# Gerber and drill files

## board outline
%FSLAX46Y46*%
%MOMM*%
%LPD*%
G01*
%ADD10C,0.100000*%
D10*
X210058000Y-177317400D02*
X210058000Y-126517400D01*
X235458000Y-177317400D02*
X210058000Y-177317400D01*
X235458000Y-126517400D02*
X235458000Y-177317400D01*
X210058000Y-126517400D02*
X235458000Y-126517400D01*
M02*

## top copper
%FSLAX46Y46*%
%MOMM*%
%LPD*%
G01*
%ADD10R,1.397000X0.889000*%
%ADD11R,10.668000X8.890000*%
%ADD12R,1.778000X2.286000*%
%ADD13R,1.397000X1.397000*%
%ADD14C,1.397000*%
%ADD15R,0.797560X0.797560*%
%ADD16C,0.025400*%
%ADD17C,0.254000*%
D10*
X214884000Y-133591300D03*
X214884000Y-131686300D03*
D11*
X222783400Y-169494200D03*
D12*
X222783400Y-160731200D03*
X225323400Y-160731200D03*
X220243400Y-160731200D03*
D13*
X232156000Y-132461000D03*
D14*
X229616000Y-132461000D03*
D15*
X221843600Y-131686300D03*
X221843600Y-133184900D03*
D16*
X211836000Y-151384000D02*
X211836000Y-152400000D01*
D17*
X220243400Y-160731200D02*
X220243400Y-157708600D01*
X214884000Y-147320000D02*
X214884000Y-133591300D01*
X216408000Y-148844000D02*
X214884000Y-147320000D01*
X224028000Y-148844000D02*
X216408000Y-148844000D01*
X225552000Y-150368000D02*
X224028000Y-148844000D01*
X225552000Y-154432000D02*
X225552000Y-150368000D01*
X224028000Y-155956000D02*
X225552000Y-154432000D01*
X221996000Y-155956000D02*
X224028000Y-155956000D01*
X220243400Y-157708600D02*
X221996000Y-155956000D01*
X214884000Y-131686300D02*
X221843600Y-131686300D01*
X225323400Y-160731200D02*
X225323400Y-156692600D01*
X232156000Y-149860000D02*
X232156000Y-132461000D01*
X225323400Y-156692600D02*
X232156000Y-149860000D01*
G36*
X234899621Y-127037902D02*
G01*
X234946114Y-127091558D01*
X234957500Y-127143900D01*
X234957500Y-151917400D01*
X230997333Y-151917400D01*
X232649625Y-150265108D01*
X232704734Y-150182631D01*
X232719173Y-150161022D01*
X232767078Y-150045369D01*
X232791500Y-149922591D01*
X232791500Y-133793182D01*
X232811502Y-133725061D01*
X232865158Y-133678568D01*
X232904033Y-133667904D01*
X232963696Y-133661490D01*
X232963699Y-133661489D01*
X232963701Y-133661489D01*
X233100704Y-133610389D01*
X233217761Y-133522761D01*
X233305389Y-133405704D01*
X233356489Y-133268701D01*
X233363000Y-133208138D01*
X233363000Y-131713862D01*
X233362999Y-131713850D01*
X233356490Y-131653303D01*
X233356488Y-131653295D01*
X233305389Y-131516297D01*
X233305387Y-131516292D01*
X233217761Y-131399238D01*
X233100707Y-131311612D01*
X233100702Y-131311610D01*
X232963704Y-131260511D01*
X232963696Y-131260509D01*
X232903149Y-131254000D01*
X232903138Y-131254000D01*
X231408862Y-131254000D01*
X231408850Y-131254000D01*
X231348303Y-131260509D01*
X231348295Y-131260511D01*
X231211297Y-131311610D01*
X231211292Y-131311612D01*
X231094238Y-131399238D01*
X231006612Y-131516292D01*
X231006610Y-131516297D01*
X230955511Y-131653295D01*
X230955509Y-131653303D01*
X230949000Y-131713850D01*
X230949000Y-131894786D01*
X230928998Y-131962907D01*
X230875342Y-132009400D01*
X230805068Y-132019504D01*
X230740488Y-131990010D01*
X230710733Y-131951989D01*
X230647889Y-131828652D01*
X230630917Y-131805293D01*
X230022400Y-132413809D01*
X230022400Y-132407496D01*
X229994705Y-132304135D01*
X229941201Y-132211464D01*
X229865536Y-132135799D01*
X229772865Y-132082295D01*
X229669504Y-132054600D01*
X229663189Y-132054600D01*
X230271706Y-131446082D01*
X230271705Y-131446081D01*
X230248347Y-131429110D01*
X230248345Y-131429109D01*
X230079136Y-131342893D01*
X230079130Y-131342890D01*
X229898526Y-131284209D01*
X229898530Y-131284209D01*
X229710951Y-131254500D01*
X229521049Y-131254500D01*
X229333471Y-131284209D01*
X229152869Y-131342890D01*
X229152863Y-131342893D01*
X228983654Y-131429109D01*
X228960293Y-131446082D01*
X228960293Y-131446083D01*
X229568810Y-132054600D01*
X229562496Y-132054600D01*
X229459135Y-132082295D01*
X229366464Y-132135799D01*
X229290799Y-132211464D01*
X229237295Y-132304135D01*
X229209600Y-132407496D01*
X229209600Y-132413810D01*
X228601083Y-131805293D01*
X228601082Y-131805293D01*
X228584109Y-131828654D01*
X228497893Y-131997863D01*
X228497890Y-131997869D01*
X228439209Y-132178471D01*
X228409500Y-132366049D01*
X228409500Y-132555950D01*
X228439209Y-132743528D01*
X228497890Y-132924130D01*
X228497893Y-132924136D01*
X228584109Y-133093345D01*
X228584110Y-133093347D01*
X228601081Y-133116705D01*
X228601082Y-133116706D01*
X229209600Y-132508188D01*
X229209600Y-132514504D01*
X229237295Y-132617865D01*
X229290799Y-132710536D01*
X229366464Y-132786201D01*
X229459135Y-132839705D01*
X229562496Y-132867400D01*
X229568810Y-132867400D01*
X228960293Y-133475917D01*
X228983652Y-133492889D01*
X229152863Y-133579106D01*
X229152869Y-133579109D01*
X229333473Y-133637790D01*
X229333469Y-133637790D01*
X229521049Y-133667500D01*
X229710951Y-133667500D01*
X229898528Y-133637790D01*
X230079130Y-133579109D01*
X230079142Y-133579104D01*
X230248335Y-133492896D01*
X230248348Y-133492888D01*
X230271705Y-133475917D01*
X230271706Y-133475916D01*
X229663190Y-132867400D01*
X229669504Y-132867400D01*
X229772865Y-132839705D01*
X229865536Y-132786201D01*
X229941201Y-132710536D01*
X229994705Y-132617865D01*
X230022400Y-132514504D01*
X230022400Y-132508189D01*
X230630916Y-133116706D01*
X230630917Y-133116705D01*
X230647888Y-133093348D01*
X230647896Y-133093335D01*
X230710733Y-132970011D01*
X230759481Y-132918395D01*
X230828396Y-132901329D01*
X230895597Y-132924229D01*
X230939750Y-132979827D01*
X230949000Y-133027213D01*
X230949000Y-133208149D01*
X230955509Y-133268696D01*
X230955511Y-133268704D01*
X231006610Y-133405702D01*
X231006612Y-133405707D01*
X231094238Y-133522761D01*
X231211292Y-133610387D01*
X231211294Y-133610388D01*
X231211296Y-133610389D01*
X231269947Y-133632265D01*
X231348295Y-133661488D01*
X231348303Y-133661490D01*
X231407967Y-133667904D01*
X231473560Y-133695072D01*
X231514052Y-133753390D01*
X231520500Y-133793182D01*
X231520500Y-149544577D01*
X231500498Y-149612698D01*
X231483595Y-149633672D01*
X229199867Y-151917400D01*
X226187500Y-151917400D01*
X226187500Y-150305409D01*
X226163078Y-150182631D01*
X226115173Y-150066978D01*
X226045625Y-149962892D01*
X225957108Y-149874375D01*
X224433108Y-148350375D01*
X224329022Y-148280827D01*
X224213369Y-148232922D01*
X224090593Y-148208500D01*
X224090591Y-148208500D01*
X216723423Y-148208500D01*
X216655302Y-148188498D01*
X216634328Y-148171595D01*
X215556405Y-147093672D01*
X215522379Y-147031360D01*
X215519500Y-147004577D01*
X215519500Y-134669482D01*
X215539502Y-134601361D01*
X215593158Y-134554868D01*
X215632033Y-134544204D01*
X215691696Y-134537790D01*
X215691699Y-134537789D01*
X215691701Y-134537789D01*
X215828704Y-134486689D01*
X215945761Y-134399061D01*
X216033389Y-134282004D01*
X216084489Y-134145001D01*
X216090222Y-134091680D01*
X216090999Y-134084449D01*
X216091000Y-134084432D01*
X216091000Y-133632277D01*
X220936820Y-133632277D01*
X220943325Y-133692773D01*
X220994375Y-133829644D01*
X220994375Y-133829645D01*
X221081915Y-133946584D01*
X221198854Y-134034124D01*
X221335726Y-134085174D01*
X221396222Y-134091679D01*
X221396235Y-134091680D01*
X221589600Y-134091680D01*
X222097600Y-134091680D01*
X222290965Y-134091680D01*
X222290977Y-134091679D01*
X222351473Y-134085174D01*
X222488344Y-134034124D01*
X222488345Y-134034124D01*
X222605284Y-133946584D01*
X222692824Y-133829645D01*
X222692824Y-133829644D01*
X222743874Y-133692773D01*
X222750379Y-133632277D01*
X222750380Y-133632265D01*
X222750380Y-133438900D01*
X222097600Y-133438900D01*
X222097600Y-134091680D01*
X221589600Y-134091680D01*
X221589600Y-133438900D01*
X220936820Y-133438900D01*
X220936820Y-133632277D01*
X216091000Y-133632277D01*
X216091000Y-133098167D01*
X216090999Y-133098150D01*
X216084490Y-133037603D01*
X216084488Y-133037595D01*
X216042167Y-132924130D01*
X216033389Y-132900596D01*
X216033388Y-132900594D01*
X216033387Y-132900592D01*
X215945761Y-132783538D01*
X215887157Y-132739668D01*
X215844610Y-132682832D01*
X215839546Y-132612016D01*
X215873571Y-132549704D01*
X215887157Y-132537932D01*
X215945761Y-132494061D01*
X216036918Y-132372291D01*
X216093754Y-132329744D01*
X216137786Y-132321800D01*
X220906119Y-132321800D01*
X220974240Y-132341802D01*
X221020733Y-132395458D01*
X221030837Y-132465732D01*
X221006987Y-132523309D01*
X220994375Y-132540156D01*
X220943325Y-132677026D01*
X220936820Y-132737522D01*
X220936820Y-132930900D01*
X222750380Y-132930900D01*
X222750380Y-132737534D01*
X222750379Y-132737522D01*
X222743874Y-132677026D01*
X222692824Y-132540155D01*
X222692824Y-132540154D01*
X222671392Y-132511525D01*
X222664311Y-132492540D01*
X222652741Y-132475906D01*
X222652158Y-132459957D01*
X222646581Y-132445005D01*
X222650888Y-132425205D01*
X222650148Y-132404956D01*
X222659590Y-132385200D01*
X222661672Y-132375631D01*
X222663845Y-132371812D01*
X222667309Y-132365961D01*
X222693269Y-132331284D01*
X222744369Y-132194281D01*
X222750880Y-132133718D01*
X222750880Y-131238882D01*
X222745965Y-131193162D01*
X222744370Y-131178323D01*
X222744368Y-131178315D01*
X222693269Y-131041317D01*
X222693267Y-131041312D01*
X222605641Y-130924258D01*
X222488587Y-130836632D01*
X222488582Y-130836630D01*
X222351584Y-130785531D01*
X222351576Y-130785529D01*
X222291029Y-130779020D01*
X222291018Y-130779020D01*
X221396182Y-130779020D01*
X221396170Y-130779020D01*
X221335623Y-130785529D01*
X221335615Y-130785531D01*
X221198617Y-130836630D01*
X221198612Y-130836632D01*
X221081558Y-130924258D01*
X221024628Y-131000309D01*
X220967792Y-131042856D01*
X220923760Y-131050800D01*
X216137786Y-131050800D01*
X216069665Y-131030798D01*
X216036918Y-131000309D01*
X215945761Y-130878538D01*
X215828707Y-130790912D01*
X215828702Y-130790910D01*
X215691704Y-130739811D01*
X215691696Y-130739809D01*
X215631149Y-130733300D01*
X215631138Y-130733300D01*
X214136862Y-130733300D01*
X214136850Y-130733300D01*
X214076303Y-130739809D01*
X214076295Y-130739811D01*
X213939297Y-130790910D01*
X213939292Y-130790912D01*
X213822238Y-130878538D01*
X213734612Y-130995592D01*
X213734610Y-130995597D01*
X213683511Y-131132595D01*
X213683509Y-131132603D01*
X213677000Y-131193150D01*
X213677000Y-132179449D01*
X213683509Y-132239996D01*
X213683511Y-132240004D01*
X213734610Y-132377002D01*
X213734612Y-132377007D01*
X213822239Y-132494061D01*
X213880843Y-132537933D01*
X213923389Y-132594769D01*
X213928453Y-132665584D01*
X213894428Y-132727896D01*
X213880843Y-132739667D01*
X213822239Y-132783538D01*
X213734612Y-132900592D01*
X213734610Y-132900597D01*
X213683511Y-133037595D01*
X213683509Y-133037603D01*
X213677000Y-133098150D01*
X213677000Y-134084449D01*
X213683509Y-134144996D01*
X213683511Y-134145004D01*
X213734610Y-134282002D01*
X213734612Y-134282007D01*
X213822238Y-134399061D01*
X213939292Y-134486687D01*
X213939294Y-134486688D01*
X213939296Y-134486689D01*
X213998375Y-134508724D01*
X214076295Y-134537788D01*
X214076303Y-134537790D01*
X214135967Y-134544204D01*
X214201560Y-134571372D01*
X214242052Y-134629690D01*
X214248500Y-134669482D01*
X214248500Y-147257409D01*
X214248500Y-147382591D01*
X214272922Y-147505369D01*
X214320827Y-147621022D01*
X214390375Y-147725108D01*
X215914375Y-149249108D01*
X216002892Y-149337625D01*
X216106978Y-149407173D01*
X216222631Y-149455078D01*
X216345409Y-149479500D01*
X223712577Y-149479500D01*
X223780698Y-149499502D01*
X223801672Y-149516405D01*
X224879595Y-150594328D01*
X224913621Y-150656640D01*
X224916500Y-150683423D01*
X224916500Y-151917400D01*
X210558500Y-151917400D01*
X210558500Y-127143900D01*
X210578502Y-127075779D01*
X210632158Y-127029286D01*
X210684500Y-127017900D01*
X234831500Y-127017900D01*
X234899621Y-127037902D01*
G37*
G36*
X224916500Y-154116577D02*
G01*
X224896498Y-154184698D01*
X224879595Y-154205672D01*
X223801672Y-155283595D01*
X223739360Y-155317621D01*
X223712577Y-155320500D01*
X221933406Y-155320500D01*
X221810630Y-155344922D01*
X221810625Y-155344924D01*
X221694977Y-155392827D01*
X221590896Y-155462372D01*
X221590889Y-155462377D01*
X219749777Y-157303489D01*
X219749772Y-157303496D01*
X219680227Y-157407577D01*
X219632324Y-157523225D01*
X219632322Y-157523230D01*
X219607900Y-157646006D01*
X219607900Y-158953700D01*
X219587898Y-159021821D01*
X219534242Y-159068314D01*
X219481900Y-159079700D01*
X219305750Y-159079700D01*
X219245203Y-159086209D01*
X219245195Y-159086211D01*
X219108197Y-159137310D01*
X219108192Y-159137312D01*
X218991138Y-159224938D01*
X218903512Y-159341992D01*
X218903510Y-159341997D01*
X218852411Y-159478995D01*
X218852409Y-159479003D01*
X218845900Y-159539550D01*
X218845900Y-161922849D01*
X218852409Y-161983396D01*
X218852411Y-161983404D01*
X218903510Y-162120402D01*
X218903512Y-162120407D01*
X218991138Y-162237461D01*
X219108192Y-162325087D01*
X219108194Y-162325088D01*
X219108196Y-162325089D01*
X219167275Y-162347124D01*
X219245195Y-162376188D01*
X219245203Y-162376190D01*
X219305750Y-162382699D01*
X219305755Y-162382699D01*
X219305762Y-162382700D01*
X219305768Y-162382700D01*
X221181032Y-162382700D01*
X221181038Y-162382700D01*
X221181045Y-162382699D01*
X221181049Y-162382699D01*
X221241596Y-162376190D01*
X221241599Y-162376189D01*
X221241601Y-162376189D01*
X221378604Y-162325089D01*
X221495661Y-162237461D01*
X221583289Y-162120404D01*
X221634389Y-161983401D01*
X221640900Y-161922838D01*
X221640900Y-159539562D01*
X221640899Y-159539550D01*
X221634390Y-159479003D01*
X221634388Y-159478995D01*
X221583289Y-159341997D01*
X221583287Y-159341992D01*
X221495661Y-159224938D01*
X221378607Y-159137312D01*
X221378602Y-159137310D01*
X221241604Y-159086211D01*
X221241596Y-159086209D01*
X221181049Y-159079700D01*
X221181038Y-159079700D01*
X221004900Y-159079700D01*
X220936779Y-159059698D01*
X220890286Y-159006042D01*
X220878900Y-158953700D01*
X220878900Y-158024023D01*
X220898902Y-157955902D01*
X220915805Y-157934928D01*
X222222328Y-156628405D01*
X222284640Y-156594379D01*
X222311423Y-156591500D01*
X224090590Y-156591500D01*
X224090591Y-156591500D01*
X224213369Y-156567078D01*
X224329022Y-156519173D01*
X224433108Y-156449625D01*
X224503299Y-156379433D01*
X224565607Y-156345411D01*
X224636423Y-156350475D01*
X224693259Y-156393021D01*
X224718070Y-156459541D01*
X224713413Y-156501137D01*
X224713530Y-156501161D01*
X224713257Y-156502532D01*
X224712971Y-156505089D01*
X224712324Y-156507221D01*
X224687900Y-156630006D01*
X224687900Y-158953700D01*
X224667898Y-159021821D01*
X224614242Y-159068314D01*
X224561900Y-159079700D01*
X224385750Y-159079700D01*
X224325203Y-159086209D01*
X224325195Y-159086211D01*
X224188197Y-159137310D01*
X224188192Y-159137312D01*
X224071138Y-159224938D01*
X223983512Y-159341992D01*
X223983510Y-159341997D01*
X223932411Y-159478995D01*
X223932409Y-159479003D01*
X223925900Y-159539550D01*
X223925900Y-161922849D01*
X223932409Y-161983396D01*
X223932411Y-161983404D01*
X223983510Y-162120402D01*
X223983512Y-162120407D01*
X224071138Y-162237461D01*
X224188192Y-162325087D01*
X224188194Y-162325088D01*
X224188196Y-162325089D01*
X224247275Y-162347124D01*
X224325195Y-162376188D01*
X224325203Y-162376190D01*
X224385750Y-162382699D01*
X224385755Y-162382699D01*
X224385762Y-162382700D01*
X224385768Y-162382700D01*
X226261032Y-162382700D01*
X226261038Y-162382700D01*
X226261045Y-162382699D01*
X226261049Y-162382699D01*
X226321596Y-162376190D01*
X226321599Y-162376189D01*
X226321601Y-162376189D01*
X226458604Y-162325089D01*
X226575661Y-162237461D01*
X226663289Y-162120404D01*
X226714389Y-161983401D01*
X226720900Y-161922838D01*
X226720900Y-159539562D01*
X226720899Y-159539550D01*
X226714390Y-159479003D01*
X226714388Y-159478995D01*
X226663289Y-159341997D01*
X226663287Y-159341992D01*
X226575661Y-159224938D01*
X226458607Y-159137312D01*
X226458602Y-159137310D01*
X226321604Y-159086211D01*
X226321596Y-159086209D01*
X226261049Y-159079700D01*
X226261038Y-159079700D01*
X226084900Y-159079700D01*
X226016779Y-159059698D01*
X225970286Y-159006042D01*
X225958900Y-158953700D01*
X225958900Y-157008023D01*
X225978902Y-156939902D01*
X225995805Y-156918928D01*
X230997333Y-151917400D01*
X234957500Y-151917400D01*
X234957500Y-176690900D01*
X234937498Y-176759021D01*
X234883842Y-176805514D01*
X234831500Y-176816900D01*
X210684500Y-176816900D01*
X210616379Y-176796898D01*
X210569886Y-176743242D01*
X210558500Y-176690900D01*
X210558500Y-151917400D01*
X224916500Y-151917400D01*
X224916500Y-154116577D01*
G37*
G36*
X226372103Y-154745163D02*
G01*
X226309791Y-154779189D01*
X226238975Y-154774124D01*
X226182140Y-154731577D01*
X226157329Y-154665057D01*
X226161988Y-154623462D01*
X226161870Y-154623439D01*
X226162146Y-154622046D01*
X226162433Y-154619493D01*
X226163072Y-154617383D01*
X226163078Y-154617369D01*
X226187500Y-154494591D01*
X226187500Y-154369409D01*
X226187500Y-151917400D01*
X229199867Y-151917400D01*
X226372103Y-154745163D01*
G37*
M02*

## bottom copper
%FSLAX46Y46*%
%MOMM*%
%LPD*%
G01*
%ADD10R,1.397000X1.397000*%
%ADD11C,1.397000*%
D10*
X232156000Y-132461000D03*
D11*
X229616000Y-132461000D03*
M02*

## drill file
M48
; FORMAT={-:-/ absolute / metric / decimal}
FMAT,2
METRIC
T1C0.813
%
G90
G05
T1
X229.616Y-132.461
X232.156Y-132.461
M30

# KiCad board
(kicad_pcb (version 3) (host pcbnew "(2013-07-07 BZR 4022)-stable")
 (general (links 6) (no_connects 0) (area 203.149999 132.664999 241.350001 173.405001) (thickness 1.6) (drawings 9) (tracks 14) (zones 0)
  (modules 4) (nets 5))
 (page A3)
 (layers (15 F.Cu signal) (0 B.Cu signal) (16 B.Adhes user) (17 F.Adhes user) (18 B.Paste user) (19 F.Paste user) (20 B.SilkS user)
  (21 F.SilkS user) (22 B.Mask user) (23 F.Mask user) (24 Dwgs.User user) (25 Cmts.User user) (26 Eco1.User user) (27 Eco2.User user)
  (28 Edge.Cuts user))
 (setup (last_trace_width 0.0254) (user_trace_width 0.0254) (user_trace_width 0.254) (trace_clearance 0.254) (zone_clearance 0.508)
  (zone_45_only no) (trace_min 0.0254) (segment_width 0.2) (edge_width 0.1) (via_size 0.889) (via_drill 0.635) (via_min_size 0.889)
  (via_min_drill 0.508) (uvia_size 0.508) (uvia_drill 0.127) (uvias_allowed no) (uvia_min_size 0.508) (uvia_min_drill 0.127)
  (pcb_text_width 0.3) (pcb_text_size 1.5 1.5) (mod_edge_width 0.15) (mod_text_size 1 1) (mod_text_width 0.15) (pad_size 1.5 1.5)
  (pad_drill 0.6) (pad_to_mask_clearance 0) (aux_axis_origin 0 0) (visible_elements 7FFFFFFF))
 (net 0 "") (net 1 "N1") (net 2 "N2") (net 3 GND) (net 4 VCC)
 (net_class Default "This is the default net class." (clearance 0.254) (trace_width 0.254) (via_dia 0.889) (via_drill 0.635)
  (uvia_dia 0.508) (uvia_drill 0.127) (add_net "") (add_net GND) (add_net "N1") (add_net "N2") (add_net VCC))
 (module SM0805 (layer F.Cu) (at 214.884 132.6388 90)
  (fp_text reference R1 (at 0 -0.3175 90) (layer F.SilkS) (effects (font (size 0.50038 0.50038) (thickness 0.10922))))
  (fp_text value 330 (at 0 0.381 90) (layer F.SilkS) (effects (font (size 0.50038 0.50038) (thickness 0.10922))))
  (pad 1 smd rect (at -0.9525 0 90) (size 0.889 1.397) (layers F.Cu F.Paste F.Mask) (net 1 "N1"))
  (pad 2 smd rect (at 0.9525 0 90) (size 0.889 1.397) (layers F.Cu F.Paste F.Mask) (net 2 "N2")))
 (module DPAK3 (layer F.Cu) (at 222.7834 160.7312 180)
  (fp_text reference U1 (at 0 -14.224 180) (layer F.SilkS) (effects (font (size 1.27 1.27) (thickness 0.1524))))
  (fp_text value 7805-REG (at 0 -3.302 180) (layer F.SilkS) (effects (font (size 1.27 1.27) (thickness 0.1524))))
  (pad 2 smd rect (at 0 -8.763 180) (size 10.668 8.89) (layers F.Cu F.Paste F.Mask) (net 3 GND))
  (pad 2 smd rect (at 0 0 180) (size 1.778 2.286) (layers F.Cu F.Paste F.Mask) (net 3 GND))
  (pad 1 smd rect (at -2.54 0 180) (size 1.778 2.286) (layers F.Cu F.Paste F.Mask) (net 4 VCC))
  (pad 3 smd rect (at 2.54 0 180) (size 1.778 2.286) (layers F.Cu F.Paste F.Mask) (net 1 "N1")))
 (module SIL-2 (layer F.Cu) (at 230.886 132.461 180)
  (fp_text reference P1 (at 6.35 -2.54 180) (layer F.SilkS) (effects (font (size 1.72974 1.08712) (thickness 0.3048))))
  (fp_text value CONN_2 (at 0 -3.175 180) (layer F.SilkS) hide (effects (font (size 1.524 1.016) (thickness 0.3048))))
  (pad 1 thru_hole rect (at -1.27 0 180) (size 1.397 1.397) (drill 0.8128) (layers *.Cu *.Mask F.SilkS) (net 4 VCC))
  (pad 2 thru_hole circle (at 1.27 0 180) (size 1.397 1.397) (drill 0.8128) (layers *.Cu *.Mask F.SilkS) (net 3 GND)))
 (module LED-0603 (layer F.Cu) (at 221.8436 132.4356 270)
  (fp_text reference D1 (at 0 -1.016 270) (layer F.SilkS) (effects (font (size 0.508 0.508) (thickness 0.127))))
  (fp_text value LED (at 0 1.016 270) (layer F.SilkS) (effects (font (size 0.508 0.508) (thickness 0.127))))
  (pad 1 smd rect (at -0.7493 0 270) (size 0.79756 0.79756) (layers F.Cu F.Paste F.Mask) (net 2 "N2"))
  (pad 2 smd rect (at 0.7493 0 270) (size 0.79756 0.79756) (layers F.Cu F.Paste F.Mask) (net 3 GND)))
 (gr_line (start 210.058 177.3174) (end 210.058 126.5174) (angle 90) (layer Edge.Cuts) (width 0.1))
 (gr_line (start 235.458 177.3174) (end 210.058 177.3174) (angle 90) (layer Edge.Cuts) (width 0.1))
 (gr_line (start 235.458 126.5174) (end 235.458 177.3174) (angle 90) (layer Edge.Cuts) (width 0.1))
 (gr_line (start 210.058 126.5174) (end 235.458 126.5174) (angle 90) (layer Edge.Cuts) (width 0.1))
 (segment (start 211.836 151.384) (end 211.836 152.4) (width 0.0254) (layer F.Cu) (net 3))
 (segment (start 220.2434 160.7312) (end 220.2434 157.7086) (width 0.254) (layer F.Cu) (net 1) (status 400000))
 (segment (start 214.884 147.32) (end 214.884 133.5913) (width 0.254) (layer F.Cu) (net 1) (status 800000))
 (segment (start 216.408 148.844) (end 214.884 147.32) (width 0.254) (layer F.Cu) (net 1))
 (segment (start 224.028 148.844) (end 216.408 148.844) (width 0.254) (layer F.Cu) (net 1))
 (segment (start 225.552 150.368) (end 224.028 148.844) (width 0.254) (layer F.Cu) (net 1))
 (segment (start 225.552 154.432) (end 225.552 150.368) (width 0.254) (layer F.Cu) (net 1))
 (segment (start 224.028 155.956) (end 225.552 154.432) (width 0.254) (layer F.Cu) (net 1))
 (segment (start 221.996 155.956) (end 224.028 155.956) (width 0.254) (layer F.Cu) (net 1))
 (segment (start 220.2434 157.7086) (end 221.996 155.956) (width 0.254) (layer F.Cu) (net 1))
 (segment (start 214.884 131.6863) (end 221.8436 131.6863) (width 0.254) (layer F.Cu) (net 2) (status C00000))
 (segment (start 225.3234 160.7312) (end 225.3234 156.6926) (width 0.254) (layer F.Cu) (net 4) (status 400000))
 (segment (start 232.156 149.86) (end 232.156 132.461) (width 0.254) (layer F.Cu) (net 4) (status 800000))
 (segment (start 225.3234 156.6926) (end 232.156 149.86) (width 0.254) (layer F.Cu) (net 4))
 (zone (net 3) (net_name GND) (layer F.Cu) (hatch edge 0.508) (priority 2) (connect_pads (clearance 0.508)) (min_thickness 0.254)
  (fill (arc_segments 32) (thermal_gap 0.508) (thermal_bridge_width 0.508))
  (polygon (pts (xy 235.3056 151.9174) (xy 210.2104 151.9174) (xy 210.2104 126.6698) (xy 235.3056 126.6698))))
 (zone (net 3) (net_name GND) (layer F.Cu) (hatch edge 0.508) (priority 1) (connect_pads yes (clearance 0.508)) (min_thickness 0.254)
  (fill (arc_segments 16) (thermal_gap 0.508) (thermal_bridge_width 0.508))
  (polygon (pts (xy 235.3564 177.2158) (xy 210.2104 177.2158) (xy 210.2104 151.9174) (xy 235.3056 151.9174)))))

